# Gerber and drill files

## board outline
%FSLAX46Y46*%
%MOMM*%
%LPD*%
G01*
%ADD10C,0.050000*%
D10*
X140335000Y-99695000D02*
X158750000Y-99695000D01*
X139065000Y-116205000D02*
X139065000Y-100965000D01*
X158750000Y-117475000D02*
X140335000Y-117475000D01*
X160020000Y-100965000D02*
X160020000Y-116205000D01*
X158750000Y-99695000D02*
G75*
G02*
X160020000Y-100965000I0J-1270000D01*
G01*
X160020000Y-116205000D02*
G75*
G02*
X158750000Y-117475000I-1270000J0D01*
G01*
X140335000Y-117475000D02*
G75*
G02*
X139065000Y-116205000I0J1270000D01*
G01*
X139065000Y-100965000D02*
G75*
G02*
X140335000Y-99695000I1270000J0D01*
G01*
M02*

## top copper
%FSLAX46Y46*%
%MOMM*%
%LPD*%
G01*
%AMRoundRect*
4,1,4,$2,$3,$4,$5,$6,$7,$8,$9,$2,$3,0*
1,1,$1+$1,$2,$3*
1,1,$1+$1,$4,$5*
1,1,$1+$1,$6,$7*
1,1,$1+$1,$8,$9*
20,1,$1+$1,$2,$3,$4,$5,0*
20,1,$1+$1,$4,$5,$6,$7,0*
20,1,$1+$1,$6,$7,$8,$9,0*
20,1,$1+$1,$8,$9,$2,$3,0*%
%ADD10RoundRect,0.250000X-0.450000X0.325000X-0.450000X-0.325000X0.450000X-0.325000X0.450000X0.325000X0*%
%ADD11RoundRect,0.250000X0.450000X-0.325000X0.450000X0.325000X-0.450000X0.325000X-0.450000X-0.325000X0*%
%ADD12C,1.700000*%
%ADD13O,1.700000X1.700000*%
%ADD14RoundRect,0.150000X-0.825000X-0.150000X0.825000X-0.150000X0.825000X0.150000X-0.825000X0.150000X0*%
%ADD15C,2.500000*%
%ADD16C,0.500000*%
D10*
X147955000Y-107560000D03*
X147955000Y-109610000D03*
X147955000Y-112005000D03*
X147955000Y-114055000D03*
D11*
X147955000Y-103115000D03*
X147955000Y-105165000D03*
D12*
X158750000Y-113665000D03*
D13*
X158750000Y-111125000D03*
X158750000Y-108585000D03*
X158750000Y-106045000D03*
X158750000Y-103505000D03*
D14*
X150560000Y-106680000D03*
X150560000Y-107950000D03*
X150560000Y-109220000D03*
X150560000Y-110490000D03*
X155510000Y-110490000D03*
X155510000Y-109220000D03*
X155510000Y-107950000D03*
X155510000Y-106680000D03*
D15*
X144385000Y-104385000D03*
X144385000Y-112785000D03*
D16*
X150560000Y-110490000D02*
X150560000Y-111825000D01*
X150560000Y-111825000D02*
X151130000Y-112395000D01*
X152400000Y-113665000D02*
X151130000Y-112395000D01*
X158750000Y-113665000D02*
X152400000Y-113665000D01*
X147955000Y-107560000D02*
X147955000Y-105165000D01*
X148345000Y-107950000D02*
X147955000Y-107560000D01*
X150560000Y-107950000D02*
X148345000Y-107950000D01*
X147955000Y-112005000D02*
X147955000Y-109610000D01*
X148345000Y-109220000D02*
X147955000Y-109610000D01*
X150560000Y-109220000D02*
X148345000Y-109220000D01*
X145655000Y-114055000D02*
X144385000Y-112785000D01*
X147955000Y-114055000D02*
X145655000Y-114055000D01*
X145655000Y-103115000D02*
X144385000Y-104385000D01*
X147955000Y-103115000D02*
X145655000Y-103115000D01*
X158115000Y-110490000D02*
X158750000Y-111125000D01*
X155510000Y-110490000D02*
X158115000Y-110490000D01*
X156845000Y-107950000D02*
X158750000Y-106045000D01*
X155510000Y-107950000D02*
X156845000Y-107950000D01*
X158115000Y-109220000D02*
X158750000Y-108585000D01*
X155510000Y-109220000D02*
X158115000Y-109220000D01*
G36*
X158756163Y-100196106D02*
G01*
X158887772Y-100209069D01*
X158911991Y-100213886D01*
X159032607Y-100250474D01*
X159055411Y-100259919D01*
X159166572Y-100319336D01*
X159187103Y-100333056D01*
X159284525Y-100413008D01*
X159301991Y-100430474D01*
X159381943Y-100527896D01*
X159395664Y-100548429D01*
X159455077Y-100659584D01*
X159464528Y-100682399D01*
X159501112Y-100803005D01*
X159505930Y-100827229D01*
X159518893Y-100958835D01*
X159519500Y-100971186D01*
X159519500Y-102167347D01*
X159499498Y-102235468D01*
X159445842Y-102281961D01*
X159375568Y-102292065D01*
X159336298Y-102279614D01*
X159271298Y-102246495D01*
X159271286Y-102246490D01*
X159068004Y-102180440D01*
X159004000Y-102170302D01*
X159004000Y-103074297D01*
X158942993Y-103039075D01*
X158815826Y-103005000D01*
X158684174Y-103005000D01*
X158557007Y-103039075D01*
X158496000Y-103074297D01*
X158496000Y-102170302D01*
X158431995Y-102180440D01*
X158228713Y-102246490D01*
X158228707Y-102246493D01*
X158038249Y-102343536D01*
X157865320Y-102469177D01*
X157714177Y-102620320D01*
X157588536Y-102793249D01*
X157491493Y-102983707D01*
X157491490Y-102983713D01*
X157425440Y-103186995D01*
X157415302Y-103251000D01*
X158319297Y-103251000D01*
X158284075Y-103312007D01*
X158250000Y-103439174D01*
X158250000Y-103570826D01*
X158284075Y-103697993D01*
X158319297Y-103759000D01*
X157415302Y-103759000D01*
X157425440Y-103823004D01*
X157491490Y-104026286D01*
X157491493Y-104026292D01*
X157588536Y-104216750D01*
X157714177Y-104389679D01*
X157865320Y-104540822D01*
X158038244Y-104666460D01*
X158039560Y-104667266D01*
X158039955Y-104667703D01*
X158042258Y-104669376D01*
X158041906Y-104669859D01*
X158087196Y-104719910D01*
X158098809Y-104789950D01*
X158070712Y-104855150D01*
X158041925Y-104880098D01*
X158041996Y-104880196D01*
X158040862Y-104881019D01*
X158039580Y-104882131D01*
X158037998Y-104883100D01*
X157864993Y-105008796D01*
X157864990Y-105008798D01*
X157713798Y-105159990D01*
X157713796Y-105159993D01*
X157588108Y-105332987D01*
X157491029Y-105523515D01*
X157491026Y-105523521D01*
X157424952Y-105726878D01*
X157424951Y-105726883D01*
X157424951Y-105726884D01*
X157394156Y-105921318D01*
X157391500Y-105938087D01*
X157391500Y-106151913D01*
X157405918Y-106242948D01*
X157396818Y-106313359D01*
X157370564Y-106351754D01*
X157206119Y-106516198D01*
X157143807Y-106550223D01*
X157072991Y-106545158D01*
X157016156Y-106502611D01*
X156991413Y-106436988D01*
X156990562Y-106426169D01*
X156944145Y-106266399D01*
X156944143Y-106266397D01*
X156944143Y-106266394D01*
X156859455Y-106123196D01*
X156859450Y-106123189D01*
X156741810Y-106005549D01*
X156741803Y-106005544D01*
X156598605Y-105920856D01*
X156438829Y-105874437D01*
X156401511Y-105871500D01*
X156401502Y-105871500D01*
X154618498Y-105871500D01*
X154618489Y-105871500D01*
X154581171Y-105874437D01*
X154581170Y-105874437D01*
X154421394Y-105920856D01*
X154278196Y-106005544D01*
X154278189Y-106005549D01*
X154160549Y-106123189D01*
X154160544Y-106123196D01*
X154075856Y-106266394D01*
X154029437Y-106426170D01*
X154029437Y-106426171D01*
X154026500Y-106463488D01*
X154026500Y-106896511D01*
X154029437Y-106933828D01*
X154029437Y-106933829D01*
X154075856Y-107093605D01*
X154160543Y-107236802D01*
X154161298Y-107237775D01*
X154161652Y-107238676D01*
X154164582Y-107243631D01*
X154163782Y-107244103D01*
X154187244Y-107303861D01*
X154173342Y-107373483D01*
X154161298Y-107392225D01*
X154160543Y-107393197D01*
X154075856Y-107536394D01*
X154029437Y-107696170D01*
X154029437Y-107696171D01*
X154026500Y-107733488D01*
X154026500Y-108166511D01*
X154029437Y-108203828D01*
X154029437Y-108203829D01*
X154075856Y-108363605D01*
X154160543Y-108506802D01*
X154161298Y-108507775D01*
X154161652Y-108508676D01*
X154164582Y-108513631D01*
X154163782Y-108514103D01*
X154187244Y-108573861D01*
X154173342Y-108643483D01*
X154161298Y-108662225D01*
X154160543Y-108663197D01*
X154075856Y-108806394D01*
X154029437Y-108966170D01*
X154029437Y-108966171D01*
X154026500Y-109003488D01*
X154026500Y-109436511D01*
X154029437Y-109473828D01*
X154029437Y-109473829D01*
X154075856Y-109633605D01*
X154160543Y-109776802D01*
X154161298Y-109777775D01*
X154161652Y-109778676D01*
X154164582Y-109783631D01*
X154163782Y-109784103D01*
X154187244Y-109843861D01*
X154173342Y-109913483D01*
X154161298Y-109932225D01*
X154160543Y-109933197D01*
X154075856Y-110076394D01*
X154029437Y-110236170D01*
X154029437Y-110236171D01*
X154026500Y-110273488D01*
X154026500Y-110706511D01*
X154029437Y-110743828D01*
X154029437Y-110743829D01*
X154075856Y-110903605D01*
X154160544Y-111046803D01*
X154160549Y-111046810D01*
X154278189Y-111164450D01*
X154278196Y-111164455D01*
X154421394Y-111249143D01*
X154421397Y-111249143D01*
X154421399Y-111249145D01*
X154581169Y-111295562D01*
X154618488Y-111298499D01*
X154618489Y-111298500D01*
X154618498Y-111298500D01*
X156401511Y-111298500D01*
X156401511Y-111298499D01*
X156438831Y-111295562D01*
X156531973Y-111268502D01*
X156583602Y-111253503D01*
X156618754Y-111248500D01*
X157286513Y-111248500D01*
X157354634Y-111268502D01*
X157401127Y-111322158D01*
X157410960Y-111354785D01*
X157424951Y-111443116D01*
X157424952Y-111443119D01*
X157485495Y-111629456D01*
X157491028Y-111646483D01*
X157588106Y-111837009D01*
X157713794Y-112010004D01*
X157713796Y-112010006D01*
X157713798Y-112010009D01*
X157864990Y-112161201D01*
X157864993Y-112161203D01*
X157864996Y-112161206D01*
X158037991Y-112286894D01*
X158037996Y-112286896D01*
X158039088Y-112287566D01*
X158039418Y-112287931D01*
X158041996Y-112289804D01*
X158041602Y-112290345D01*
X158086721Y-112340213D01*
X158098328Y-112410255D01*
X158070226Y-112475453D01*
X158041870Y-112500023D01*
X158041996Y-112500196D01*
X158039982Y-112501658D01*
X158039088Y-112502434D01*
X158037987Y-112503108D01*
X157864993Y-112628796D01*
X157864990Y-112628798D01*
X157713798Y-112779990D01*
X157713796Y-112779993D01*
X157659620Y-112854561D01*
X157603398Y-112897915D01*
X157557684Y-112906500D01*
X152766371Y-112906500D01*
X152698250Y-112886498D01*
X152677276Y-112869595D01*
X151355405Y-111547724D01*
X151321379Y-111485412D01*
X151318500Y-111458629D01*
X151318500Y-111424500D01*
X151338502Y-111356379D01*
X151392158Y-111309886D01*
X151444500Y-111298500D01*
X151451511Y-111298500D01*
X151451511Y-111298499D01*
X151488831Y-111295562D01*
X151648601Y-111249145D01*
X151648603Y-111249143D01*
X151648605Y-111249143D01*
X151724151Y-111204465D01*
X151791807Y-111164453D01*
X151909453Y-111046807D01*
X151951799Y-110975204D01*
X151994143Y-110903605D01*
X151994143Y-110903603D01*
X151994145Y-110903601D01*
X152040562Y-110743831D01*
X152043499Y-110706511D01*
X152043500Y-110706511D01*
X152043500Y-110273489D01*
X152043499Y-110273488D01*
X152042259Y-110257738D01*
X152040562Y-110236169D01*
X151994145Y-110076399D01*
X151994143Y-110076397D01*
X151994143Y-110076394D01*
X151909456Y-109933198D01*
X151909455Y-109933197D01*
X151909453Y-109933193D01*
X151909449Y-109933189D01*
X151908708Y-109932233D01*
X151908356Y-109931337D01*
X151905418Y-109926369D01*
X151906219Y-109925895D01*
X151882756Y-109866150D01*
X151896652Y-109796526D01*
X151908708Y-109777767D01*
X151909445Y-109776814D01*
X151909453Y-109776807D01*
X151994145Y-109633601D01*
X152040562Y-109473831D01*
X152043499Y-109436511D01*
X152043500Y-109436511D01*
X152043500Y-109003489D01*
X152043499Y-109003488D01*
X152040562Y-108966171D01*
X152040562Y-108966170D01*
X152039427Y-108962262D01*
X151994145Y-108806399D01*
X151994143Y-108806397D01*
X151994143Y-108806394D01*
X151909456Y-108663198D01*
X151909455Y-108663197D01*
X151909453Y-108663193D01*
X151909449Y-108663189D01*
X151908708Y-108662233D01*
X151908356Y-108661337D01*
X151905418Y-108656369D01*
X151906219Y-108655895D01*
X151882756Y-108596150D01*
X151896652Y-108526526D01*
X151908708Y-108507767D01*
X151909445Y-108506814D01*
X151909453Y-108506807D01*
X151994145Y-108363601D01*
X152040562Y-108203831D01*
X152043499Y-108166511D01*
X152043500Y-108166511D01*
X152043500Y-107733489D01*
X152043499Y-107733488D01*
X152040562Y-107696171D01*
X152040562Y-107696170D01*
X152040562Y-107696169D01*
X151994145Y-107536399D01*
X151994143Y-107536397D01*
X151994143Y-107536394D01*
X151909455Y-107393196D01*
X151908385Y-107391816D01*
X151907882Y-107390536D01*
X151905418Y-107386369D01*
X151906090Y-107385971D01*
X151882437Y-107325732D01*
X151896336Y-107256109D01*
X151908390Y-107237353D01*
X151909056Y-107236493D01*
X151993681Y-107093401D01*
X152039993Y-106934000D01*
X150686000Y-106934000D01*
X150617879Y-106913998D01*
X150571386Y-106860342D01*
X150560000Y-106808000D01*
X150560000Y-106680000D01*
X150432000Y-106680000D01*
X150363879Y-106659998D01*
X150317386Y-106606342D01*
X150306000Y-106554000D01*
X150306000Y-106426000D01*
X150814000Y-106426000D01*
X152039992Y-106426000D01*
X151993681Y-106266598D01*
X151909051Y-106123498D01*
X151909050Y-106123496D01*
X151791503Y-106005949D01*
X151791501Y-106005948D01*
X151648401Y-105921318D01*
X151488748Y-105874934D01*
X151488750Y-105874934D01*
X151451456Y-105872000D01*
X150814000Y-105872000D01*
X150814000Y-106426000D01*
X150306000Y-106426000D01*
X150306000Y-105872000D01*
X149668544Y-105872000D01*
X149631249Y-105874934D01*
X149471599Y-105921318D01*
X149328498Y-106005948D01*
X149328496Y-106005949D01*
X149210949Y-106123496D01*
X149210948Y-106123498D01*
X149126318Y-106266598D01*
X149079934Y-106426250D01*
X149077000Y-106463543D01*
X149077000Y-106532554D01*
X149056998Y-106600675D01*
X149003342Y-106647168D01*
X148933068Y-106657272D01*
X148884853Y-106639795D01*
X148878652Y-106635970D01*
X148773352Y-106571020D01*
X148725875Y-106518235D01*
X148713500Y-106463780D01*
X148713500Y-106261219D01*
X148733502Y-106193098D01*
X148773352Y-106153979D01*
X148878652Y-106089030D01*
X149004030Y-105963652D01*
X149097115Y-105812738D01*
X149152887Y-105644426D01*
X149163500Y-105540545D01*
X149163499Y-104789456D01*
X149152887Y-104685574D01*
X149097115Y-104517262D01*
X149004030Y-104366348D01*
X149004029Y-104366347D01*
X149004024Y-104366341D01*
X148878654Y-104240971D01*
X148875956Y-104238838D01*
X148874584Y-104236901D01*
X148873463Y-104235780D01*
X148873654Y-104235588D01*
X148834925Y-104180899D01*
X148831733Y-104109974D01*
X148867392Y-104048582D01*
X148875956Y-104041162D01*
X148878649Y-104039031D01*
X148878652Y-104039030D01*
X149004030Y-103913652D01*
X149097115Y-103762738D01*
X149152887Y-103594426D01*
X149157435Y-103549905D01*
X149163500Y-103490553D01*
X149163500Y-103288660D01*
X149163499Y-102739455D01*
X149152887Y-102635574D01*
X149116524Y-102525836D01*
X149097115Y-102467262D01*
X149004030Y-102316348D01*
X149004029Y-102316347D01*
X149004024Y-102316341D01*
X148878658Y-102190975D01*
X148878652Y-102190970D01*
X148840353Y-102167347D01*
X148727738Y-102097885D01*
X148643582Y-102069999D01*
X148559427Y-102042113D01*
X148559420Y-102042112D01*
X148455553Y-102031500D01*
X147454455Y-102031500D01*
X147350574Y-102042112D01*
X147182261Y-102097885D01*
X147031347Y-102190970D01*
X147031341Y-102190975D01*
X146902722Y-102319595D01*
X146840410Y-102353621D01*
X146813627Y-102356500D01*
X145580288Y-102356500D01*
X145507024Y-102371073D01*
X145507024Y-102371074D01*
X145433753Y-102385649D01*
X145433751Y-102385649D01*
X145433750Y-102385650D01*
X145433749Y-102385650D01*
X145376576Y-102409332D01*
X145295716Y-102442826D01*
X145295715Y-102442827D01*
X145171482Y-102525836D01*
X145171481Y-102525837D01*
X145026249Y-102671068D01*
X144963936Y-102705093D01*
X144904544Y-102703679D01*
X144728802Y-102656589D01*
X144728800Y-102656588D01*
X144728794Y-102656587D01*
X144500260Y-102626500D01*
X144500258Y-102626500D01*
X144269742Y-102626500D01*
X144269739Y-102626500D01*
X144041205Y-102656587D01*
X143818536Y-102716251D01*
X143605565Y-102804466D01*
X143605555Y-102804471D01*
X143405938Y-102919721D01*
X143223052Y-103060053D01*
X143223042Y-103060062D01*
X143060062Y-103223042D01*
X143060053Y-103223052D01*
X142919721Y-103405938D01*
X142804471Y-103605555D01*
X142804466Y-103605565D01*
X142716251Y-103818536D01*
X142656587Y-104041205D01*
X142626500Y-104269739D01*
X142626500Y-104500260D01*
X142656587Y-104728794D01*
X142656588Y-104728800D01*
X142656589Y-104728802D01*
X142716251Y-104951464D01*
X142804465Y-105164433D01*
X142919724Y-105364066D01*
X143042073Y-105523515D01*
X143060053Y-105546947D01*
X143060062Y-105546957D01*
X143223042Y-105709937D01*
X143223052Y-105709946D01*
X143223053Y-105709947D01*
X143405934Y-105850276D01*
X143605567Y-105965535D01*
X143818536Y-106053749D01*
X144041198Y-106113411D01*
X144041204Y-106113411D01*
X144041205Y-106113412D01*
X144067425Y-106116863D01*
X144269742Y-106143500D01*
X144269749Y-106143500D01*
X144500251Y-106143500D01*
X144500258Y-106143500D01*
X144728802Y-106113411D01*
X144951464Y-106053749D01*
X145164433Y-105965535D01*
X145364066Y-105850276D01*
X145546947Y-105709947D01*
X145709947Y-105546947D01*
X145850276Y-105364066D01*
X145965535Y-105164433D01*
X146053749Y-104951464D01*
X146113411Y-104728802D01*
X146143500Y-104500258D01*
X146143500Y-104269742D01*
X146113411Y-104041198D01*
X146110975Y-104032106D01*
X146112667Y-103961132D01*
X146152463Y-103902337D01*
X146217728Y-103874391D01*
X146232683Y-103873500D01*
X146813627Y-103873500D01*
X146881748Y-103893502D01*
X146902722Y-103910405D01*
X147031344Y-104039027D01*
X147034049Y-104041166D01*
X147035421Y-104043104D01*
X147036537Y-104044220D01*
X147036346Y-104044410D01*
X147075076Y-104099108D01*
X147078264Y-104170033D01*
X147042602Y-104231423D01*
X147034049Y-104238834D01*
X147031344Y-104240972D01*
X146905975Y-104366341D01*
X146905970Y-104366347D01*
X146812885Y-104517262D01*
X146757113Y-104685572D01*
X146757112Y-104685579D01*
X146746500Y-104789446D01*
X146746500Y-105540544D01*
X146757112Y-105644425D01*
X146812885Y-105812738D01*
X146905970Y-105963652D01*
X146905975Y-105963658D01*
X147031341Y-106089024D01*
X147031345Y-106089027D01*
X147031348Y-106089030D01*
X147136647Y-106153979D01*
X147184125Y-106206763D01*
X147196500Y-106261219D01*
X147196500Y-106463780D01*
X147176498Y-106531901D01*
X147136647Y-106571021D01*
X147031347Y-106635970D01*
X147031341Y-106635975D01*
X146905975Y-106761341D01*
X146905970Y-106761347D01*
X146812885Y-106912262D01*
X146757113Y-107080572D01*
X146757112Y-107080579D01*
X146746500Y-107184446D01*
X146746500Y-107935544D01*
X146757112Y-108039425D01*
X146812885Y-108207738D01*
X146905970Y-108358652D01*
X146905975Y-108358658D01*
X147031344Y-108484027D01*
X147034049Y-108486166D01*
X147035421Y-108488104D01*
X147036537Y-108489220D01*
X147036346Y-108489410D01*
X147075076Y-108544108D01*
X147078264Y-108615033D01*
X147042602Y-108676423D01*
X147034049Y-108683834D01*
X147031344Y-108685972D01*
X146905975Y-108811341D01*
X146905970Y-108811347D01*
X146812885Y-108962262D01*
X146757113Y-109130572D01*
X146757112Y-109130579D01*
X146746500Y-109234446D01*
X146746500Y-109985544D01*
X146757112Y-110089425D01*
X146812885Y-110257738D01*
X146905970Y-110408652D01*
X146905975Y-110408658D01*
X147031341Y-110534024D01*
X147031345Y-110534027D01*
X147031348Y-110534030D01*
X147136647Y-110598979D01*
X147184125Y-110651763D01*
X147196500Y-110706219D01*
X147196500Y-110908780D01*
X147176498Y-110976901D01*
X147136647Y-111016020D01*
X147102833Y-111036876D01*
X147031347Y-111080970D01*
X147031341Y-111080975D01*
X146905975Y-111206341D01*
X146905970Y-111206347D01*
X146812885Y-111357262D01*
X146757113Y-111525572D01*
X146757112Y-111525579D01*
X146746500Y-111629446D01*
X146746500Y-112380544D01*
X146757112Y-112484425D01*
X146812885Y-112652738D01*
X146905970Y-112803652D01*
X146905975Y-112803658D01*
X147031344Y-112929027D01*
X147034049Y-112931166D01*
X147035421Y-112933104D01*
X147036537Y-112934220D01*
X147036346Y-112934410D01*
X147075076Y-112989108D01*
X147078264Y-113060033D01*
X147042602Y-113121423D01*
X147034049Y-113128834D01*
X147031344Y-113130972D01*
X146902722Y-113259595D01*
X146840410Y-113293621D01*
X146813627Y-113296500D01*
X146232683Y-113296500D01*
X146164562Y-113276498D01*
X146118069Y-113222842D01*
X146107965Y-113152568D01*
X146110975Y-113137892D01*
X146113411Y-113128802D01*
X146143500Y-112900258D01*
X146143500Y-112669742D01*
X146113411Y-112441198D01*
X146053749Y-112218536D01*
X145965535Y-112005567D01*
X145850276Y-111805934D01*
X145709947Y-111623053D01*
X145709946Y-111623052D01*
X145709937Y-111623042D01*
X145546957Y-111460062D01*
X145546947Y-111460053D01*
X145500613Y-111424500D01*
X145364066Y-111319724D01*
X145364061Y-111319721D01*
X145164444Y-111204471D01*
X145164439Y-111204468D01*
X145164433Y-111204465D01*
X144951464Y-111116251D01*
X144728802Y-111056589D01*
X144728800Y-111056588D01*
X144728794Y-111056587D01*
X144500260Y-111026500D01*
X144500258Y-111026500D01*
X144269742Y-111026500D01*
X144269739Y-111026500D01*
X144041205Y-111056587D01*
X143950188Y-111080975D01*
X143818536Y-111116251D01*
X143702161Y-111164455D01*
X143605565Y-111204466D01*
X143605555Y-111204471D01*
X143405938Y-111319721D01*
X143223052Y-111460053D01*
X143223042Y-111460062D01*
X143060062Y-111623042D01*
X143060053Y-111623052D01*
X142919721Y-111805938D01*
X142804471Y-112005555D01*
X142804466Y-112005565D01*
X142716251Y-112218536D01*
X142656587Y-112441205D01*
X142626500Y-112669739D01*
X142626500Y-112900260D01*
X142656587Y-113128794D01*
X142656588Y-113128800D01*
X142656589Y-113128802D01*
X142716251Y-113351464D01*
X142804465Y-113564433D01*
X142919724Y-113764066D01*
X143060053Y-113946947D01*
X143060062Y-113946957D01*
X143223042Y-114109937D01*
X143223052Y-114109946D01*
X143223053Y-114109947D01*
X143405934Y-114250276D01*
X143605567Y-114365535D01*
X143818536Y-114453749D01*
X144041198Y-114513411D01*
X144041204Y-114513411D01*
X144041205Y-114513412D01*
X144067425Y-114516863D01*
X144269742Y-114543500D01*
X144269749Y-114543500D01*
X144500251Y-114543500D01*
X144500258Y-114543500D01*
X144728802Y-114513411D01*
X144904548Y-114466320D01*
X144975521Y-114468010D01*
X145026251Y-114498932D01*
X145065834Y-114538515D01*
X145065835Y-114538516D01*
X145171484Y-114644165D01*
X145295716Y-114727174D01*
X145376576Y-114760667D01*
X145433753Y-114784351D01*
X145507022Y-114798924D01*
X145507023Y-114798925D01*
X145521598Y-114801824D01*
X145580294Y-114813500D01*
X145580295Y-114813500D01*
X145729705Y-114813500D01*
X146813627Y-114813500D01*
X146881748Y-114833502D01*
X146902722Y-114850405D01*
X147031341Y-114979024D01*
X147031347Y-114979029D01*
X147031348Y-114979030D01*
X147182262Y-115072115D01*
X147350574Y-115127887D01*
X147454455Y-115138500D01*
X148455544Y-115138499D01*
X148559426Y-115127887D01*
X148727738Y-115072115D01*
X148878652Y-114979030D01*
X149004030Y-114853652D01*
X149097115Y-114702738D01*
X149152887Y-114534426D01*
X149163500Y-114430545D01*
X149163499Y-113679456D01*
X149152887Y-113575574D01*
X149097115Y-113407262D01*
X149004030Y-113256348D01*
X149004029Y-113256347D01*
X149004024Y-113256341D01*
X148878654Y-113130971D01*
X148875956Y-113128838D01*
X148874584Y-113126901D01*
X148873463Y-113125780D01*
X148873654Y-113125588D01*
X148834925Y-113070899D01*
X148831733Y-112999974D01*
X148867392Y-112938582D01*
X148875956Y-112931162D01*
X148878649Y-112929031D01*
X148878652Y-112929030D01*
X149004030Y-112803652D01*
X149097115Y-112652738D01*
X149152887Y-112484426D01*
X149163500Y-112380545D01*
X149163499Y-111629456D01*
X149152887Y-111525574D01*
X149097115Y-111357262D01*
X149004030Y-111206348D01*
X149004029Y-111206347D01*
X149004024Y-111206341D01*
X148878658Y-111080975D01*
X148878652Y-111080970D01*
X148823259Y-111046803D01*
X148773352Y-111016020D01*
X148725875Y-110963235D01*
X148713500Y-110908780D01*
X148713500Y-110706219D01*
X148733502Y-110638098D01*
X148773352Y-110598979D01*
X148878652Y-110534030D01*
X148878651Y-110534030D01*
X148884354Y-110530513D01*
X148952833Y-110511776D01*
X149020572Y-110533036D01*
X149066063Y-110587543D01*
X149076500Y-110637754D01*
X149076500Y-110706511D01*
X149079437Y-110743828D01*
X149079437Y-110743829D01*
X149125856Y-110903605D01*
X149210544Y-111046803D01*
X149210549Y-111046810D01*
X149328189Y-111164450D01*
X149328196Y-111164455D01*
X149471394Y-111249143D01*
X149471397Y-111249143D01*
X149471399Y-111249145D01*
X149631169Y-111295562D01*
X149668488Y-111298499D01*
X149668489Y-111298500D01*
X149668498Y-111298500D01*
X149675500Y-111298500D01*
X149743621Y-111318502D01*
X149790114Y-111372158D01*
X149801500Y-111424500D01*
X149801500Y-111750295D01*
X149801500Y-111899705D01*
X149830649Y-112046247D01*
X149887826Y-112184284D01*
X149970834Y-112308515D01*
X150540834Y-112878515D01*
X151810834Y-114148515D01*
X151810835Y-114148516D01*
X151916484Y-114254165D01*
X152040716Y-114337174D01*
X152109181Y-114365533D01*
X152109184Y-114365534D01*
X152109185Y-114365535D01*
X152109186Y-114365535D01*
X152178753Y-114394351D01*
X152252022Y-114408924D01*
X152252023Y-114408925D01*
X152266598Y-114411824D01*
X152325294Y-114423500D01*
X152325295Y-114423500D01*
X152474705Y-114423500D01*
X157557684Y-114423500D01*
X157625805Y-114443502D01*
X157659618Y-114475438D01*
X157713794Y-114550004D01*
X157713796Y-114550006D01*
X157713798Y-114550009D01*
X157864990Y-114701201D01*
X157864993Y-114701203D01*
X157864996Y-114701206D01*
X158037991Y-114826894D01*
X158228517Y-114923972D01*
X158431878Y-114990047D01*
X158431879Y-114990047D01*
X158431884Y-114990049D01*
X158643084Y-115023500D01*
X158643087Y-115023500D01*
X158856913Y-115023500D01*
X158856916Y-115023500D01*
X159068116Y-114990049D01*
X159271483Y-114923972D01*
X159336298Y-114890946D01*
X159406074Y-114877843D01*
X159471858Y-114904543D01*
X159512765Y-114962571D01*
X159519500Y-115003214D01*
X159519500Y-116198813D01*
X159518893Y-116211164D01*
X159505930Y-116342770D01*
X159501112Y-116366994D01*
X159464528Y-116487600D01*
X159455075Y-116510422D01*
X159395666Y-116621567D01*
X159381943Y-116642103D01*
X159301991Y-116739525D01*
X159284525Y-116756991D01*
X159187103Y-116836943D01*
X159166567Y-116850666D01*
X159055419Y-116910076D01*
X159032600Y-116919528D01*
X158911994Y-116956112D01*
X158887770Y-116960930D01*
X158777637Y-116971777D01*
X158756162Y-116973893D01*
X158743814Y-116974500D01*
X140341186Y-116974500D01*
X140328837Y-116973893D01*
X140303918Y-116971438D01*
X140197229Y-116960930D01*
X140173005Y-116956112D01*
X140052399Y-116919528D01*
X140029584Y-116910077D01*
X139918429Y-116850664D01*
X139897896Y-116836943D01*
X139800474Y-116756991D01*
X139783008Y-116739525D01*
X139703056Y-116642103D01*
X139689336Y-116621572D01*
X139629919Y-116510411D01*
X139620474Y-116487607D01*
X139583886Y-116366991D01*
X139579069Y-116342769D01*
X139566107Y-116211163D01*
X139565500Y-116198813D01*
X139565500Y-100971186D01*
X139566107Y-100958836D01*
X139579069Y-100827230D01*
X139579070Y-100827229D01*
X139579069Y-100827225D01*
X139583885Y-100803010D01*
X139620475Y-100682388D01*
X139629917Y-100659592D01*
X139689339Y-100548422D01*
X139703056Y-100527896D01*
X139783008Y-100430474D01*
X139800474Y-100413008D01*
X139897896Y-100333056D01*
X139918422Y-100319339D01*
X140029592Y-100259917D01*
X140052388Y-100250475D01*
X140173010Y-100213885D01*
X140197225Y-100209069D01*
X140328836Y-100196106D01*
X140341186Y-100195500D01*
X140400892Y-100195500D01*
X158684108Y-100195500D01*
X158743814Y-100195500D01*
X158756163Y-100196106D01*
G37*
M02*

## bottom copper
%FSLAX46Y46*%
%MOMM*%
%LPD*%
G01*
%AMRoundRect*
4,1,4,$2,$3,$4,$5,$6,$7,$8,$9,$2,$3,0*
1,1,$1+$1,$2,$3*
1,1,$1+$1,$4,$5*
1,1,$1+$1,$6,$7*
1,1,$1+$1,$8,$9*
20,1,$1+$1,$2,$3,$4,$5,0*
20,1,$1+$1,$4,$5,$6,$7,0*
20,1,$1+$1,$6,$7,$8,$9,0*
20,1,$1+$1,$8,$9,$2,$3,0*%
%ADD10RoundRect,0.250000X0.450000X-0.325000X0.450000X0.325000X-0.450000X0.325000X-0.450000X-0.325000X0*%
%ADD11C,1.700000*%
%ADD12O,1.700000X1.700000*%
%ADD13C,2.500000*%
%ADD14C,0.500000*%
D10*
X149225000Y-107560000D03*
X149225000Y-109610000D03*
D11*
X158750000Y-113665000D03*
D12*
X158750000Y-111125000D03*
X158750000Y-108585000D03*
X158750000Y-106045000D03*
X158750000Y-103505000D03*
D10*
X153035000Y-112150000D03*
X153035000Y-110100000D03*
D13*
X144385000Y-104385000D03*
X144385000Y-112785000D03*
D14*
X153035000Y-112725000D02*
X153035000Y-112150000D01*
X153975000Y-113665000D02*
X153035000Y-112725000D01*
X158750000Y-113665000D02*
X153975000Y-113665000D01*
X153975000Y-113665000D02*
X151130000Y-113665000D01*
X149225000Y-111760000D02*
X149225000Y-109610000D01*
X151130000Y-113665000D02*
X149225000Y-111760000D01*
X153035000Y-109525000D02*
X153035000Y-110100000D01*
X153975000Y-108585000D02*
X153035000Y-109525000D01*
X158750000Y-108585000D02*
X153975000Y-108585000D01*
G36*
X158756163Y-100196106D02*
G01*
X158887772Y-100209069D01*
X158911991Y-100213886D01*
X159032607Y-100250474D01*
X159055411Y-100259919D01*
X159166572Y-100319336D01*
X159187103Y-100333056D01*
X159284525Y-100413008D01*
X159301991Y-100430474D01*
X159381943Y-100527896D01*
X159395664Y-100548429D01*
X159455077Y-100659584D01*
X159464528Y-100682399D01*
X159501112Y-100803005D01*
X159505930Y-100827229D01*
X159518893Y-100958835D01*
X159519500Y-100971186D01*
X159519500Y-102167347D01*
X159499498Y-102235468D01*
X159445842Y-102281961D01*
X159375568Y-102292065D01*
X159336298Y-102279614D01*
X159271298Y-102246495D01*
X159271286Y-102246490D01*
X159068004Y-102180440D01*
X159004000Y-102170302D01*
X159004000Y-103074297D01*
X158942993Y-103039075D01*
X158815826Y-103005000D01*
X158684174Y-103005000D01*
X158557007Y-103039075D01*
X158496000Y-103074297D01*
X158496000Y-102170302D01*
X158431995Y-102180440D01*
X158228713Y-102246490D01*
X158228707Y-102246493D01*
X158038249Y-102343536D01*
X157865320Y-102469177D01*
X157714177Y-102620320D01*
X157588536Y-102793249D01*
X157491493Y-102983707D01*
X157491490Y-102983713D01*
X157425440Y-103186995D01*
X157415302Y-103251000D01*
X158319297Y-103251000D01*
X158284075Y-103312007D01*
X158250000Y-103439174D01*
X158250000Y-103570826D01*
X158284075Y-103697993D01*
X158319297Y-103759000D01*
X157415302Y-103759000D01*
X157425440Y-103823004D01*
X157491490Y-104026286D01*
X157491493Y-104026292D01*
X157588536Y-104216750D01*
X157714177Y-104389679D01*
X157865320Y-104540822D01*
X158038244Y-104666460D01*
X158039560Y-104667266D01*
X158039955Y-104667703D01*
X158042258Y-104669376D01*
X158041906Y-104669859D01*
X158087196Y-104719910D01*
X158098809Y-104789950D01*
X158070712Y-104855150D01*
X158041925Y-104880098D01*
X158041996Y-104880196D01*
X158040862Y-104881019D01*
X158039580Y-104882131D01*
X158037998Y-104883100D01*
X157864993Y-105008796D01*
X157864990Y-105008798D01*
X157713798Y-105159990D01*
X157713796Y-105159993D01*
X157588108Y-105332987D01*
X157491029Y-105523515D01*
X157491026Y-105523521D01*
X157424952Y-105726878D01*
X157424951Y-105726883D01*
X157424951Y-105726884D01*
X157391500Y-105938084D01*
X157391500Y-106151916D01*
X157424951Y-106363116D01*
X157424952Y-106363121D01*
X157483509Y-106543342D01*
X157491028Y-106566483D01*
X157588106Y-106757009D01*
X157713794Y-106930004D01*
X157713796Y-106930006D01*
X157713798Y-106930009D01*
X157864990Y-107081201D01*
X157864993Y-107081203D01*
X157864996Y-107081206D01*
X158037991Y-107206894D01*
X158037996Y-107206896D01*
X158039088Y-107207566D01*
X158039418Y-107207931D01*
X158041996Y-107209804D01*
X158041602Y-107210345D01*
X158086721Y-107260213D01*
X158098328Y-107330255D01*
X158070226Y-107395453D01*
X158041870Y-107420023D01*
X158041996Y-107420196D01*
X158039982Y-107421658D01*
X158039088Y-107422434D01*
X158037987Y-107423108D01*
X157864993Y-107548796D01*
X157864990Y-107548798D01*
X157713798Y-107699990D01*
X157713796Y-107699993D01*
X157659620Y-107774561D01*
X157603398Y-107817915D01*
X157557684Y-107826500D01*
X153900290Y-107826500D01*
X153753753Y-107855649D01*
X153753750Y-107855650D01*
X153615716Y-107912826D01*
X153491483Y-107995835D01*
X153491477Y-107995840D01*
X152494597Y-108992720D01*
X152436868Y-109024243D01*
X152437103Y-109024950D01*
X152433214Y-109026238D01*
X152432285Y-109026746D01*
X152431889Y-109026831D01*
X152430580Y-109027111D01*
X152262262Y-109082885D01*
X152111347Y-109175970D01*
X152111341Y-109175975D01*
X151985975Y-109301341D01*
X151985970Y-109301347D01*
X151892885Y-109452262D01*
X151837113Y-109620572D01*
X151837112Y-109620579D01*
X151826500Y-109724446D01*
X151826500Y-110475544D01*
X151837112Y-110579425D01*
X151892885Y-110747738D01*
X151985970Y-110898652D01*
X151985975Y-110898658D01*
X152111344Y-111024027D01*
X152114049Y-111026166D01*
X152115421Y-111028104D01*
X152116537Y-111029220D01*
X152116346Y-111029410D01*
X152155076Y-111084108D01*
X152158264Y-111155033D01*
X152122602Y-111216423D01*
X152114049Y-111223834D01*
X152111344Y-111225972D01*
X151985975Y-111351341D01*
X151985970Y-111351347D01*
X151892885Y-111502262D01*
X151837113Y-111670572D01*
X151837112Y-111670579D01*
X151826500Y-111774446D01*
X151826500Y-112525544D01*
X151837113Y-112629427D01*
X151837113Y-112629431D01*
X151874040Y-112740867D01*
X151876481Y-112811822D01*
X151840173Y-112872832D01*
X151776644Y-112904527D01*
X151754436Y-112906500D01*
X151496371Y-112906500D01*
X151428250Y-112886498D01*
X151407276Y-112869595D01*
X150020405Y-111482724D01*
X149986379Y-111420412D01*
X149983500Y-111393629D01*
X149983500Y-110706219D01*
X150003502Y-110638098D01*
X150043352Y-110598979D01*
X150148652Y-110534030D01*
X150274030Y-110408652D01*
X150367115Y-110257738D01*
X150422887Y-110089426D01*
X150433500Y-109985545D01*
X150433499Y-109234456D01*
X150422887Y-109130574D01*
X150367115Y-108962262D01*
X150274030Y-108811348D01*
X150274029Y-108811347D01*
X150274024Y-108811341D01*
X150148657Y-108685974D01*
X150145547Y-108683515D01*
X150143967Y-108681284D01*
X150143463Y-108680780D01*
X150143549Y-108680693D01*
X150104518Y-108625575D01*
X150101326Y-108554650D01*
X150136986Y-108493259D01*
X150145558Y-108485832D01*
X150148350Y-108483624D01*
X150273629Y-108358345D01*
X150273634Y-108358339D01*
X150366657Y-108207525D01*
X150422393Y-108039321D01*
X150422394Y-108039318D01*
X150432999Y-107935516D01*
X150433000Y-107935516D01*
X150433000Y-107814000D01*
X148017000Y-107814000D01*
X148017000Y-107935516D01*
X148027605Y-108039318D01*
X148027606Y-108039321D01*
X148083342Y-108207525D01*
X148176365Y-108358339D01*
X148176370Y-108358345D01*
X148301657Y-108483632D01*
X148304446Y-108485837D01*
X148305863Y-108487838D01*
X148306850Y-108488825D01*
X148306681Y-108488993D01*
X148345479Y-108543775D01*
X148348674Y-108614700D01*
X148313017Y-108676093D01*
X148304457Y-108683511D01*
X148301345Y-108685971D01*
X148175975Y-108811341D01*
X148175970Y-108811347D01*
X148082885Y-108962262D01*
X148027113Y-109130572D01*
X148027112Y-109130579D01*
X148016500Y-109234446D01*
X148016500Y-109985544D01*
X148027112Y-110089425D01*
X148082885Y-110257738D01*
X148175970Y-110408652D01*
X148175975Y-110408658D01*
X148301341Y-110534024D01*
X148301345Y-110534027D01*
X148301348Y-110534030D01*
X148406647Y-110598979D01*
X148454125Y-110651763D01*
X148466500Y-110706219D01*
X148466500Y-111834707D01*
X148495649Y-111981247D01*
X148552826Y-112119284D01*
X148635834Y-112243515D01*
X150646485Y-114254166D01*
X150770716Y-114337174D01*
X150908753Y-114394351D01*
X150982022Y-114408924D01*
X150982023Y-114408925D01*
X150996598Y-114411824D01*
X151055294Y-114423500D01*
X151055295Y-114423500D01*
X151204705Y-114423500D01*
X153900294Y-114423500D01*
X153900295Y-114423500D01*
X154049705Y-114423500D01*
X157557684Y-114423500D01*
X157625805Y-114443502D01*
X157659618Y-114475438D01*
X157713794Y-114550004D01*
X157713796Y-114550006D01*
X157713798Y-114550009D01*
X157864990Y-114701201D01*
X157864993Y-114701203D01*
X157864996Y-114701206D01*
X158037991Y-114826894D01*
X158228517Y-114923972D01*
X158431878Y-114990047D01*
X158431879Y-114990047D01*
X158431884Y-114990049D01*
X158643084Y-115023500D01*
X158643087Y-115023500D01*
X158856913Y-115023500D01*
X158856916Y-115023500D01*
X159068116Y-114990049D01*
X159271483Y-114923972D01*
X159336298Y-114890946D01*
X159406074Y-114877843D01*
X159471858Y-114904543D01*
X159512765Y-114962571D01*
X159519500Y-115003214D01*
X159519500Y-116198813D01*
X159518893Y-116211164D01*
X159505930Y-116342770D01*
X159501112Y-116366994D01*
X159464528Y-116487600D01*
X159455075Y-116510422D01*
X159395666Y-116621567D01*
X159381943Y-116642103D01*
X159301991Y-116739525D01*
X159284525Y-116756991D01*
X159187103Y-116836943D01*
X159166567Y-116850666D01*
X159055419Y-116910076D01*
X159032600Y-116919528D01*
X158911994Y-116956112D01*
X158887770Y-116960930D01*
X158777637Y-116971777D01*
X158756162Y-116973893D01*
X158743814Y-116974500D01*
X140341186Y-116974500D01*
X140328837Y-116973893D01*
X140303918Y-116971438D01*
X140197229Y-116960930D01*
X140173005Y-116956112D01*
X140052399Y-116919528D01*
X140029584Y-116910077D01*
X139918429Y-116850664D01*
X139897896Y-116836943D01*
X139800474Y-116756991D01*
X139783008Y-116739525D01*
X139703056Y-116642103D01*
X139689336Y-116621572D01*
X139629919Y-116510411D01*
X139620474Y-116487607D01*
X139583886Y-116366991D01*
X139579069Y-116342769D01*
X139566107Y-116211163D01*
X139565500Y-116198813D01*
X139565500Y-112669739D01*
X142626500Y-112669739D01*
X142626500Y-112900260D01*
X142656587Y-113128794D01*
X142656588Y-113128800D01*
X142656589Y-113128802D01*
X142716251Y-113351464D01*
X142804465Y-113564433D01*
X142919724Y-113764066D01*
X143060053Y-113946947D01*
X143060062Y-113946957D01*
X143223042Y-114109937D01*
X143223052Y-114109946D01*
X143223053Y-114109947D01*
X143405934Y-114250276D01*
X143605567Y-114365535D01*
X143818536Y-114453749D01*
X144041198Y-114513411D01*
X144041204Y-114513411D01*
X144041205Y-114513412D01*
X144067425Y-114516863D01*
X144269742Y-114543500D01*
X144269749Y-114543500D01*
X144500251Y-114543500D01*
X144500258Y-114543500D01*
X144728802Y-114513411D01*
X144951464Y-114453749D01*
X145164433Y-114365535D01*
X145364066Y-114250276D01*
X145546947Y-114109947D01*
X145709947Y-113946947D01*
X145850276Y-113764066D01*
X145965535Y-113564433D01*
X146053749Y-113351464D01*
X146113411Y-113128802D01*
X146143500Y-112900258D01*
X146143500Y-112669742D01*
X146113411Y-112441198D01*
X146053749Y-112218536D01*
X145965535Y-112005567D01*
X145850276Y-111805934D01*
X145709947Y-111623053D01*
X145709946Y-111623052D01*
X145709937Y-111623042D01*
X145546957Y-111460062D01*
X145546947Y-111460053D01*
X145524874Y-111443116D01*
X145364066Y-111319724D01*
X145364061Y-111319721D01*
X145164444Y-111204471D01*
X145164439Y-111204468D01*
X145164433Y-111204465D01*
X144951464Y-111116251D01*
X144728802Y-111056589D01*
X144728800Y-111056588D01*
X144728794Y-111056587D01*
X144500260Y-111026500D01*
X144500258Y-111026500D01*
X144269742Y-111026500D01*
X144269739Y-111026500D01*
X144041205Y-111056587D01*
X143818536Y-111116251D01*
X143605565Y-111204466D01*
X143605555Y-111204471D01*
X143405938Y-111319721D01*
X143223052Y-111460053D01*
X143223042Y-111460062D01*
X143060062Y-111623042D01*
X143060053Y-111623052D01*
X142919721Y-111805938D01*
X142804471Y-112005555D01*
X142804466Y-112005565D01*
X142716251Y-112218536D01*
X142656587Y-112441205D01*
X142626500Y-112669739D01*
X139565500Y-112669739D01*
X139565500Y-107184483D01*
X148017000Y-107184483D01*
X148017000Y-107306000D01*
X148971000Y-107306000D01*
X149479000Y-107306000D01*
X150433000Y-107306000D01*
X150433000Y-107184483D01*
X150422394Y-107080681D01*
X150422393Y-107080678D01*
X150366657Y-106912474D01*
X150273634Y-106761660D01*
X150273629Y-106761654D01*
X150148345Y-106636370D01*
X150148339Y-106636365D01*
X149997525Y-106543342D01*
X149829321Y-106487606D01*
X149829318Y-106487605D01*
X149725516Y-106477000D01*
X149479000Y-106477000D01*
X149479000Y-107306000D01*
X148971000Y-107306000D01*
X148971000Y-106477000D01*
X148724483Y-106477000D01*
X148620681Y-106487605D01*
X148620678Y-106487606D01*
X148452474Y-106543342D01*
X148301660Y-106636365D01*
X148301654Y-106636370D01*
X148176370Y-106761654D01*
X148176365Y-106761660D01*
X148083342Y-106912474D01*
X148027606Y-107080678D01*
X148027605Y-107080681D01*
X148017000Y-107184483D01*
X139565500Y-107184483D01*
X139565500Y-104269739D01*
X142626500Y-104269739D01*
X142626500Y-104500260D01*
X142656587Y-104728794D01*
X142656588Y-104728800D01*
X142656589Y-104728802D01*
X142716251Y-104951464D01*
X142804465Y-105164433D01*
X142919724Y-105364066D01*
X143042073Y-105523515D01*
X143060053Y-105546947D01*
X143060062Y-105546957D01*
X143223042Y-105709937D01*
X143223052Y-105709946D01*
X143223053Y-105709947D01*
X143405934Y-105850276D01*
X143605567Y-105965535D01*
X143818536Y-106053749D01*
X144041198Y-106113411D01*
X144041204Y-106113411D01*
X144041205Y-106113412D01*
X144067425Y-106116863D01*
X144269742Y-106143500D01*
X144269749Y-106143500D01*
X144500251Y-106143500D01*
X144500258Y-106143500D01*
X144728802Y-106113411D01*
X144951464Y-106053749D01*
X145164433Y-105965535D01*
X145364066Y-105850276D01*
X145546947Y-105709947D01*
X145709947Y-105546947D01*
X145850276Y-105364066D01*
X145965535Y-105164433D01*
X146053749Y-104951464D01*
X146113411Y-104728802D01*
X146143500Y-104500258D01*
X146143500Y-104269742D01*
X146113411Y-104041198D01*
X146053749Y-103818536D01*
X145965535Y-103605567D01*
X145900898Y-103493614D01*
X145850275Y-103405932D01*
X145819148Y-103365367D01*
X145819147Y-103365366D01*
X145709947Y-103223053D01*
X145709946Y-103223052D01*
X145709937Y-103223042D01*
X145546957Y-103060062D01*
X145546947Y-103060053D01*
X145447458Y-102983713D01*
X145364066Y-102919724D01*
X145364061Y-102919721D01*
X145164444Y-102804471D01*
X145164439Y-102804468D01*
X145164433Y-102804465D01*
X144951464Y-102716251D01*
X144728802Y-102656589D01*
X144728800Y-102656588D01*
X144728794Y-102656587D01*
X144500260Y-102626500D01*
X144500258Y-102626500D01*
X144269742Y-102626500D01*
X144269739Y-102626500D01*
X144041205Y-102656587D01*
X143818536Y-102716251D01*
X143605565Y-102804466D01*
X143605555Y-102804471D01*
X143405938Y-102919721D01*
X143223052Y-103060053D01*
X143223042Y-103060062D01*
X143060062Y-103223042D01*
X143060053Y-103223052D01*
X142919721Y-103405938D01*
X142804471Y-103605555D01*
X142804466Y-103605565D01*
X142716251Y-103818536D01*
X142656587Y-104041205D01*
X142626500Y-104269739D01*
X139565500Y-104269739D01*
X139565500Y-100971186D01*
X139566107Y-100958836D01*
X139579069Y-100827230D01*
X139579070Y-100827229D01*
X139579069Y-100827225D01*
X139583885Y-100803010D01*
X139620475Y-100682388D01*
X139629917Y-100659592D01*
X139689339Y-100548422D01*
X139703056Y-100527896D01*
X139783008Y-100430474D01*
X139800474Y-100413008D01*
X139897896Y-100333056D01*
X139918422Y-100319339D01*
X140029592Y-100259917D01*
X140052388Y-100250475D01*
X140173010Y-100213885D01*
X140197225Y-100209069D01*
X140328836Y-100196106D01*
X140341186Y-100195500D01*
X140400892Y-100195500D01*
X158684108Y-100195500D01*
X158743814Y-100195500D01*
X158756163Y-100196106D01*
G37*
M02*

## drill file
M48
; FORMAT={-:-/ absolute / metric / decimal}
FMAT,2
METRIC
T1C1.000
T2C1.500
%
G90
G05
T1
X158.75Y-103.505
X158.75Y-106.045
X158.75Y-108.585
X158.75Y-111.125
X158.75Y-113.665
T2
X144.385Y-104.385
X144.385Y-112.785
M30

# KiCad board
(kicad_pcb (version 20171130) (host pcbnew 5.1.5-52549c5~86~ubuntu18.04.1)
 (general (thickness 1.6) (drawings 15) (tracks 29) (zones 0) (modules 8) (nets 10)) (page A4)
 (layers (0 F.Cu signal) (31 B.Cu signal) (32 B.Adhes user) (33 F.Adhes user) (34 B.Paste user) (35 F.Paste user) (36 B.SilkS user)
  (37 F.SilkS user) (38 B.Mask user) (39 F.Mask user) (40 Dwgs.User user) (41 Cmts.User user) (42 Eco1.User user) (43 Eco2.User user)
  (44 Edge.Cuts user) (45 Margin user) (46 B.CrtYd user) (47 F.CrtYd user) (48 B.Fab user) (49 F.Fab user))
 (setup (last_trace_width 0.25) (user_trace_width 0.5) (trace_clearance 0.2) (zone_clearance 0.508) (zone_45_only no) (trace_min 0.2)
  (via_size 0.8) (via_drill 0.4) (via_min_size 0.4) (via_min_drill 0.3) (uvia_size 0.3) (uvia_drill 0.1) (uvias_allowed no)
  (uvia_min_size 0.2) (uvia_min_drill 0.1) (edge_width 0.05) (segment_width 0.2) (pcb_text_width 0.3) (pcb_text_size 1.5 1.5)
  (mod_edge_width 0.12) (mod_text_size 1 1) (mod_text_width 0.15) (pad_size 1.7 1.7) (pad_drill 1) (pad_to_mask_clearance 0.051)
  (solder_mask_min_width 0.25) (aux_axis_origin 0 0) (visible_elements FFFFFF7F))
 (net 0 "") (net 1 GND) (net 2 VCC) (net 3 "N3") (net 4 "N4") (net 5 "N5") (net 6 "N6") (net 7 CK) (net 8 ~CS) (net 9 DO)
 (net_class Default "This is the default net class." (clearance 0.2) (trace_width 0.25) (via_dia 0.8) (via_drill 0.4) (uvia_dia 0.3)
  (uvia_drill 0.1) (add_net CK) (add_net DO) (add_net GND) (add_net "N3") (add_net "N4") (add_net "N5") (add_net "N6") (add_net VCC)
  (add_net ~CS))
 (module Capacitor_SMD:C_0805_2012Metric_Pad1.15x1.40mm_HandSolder (layer B.Cu) (at 149.225 108.585 90)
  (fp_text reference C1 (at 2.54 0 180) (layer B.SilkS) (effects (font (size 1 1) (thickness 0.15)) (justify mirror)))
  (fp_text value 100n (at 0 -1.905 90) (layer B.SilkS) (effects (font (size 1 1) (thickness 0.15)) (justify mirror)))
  (pad 2 smd roundrect (at 1.025 0 90) (size 1.15 1.4) (layers B.Cu B.Paste B.Mask) (roundrect_rratio 0.217391) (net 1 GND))
  (pad 1 smd roundrect (at -1.025 0 90) (size 1.15 1.4) (layers B.Cu B.Paste B.Mask) (roundrect_rratio 0.217391) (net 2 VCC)))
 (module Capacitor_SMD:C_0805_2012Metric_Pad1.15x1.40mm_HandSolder (layer F.Cu) (at 147.955 108.585 270)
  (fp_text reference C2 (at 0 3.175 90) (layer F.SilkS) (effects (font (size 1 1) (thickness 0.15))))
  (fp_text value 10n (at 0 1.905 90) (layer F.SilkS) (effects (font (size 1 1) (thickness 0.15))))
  (pad 1 smd roundrect (at -1.025 0 270) (size 1.15 1.4) (layers F.Cu F.Paste F.Mask) (roundrect_rratio 0.217391) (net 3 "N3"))
  (pad 2 smd roundrect (at 1.025 0 270) (size 1.15 1.4) (layers F.Cu F.Paste F.Mask) (roundrect_rratio 0.217391) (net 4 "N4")))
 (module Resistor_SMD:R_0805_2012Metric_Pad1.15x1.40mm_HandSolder (layer F.Cu) (at 147.955 113.03 270)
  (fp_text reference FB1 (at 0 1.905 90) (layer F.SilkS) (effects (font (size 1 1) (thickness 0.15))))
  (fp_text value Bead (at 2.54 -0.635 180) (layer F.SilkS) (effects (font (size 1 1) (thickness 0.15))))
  (pad 1 smd roundrect (at -1.025 0 270) (size 1.15 1.4) (layers F.Cu F.Paste F.Mask) (roundrect_rratio 0.217391) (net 4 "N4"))
  (pad 2 smd roundrect (at 1.025 0 270) (size 1.15 1.4) (layers F.Cu F.Paste F.Mask) (roundrect_rratio 0.217391) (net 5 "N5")))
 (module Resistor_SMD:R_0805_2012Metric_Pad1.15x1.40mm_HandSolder (layer F.Cu) (at 147.955 104.14 90)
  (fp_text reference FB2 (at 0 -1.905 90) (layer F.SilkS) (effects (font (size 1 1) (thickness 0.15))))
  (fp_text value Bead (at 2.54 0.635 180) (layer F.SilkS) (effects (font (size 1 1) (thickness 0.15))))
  (pad 2 smd roundrect (at 1.025 0 90) (size 1.15 1.4) (layers F.Cu F.Paste F.Mask) (roundrect_rratio 0.217391) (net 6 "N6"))
  (pad 1 smd roundrect (at -1.025 0 90) (size 1.15 1.4) (layers F.Cu F.Paste F.Mask) (roundrect_rratio 0.217391) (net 3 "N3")))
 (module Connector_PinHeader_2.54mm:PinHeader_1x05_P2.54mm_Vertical (layer F.Cu) (at 158.75 113.665 180)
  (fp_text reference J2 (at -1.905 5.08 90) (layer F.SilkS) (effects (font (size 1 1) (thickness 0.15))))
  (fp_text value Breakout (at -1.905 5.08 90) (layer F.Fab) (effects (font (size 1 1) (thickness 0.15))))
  (pad 1 thru_hole circle (at 0 0 180) (size 1.7 1.7) (drill 1) (layers *.Cu *.Mask) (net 2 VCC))
  (pad 2 thru_hole oval (at 0 2.54 180) (size 1.7 1.7) (drill 1) (layers *.Cu *.Mask) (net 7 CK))
  (pad 3 thru_hole oval (at 0 5.08 180) (size 1.7 1.7) (drill 1) (layers *.Cu *.Mask) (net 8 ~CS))
  (pad 4 thru_hole oval (at 0 7.62 180) (size 1.7 1.7) (drill 1) (layers *.Cu *.Mask) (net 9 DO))
  (pad 5 thru_hole oval (at 0 10.16 180) (size 1.7 1.7) (drill 1) (layers *.Cu *.Mask) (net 1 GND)))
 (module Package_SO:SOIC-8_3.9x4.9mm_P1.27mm (layer F.Cu) (at 153.035 108.585)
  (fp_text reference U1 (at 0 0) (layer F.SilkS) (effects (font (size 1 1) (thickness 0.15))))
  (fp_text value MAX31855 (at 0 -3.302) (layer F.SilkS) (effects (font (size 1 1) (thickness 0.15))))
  (pad 1 smd roundrect (at -2.475 -1.905) (size 1.95 0.6) (layers F.Cu F.Paste F.Mask) (roundrect_rratio 0.25) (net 1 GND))
  (pad 2 smd roundrect (at -2.475 -0.635) (size 1.95 0.6) (layers F.Cu F.Paste F.Mask) (roundrect_rratio 0.25) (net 3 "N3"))
  (pad 3 smd roundrect (at -2.475 0.635) (size 1.95 0.6) (layers F.Cu F.Paste F.Mask) (roundrect_rratio 0.25) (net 4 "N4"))
  (pad 4 smd roundrect (at -2.475 1.905) (size 1.95 0.6) (layers F.Cu F.Paste F.Mask) (roundrect_rratio 0.25) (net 2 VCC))
  (pad 5 smd roundrect (at 2.475 1.905) (size 1.95 0.6) (layers F.Cu F.Paste F.Mask) (roundrect_rratio 0.25) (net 7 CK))
  (pad 6 smd roundrect (at 2.475 0.635) (size 1.95 0.6) (layers F.Cu F.Paste F.Mask) (roundrect_rratio 0.25) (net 8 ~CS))
  (pad 7 smd roundrect (at 2.475 -0.635) (size 1.95 0.6) (layers F.Cu F.Paste F.Mask) (roundrect_rratio 0.25) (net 9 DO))
  (pad 8 smd roundrect (at 2.475 -1.905) (size 1.95 0.6) (layers F.Cu F.Paste F.Mask) (roundrect_rratio 0.25)))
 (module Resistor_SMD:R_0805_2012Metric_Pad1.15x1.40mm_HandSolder (layer B.Cu) (at 153.035 111.125 90)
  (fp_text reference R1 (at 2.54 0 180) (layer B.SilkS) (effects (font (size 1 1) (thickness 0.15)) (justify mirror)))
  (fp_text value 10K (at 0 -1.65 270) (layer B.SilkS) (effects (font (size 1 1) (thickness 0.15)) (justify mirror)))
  (pad 1 smd roundrect (at -1.025 0 90) (size 1.15 1.4) (layers B.Cu B.Paste B.Mask) (roundrect_rratio 0.217391) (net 2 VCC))
  (pad 2 smd roundrect (at 1.025 0 90) (size 1.15 1.4) (layers B.Cu B.Paste B.Mask) (roundrect_rratio 0.217391) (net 8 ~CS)))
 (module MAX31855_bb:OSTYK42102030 (layer F.Cu) (at 140.335 108.585 270)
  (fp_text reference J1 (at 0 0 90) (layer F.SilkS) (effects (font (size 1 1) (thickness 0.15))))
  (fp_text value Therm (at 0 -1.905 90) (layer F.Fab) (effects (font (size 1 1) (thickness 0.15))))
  (pad 1 thru_hole circle (at -4.2 -4.05 270) (size 2.5 2.5) (drill 1.5) (layers *.Cu *.Mask) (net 6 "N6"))
  (pad 2 thru_hole circle (at 4.2 -4.05 270) (size 2.5 2.5) (drill 1.5) (layers *.Cu *.Mask) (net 5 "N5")))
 (gr_line (start 140.335 99.695) (end 158.75 99.695) (layer Edge.Cuts) (width 0.05))
 (gr_line (start 139.065 116.205) (end 139.065 100.965) (layer Edge.Cuts) (width 0.05))
 (gr_line (start 158.75 117.475) (end 140.335 117.475) (layer Edge.Cuts) (width 0.05))
 (gr_line (start 160.02 100.965) (end 160.02 116.205) (layer Edge.Cuts) (width 0.05))
 (gr_arc (start 158.75 100.965) (end 160.02 100.965) (angle -90) (layer Edge.Cuts) (width 0.05))
 (gr_arc (start 158.75 116.205) (end 158.75 117.475) (angle -90) (layer Edge.Cuts) (width 0.05))
 (gr_arc (start 140.335 116.205) (end 139.065 116.205) (angle -90) (layer Edge.Cuts) (width 0.05))
 (gr_arc (start 140.335 100.965) (end 140.335 99.695) (angle -90) (layer Edge.Cuts) (width 0.05))
 (segment (start 150.56 110.49) (end 150.56 111.825) (width 0.5) (layer F.Cu) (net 2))
 (segment (start 150.56 111.825) (end 151.13 112.395) (width 0.5) (layer F.Cu) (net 2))
 (segment (start 152.4 113.665) (end 151.13 112.395) (width 0.5) (layer F.Cu) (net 2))
 (segment (start 158.75 113.665) (end 152.4 113.665) (width 0.5) (layer F.Cu) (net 2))
 (segment (start 153.035 112.725) (end 153.035 112.15) (width 0.5) (layer B.Cu) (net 2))
 (segment (start 153.975 113.665) (end 153.035 112.725) (width 0.5) (layer B.Cu) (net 2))
 (segment (start 158.75 113.665) (end 153.975 113.665) (width 0.5) (layer B.Cu) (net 2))
 (segment (start 153.975 113.665) (end 151.13 113.665) (width 0.5) (layer B.Cu) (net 2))
 (segment (start 149.225 111.76) (end 149.225 109.61) (width 0.5) (layer B.Cu) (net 2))
 (segment (start 151.13 113.665) (end 149.225 111.76) (width 0.5) (layer B.Cu) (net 2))
 (segment (start 147.955 107.56) (end 147.955 105.165) (width 0.5) (layer F.Cu) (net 3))
 (segment (start 148.345 107.95) (end 147.955 107.56) (width 0.5) (layer F.Cu) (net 3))
 (segment (start 150.56 107.95) (end 148.345 107.95) (width 0.5) (layer F.Cu) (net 3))
 (segment (start 147.955 112.005) (end 147.955 109.61) (width 0.5) (layer F.Cu) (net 4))
 (segment (start 148.345 109.22) (end 147.955 109.61) (width 0.5) (layer F.Cu) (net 4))
 (segment (start 150.56 109.22) (end 148.345 109.22) (width 0.5) (layer F.Cu) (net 4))
 (segment (start 145.655 114.055) (end 144.385 112.785) (width 0.5) (layer F.Cu) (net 5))
 (segment (start 147.955 114.055) (end 145.655 114.055) (width 0.5) (layer F.Cu) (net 5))
 (segment (start 145.655 103.115) (end 144.385 104.385) (width 0.5) (layer F.Cu) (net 6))
 (segment (start 147.955 103.115) (end 145.655 103.115) (width 0.5) (layer F.Cu) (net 6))
 (segment (start 158.115 110.49) (end 158.75 111.125) (width 0.5) (layer F.Cu) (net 7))
 (segment (start 155.51 110.49) (end 158.115 110.49) (width 0.5) (layer F.Cu) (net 7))
 (segment (start 156.845 107.95) (end 158.75 106.045) (width 0.5) (layer F.Cu) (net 9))
 (segment (start 155.51 107.95) (end 156.845 107.95) (width 0.5) (layer F.Cu) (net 9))
 (segment (start 158.115 109.22) (end 158.75 108.585) (width 0.5) (layer F.Cu) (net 8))
 (segment (start 155.51 109.22) (end 158.115 109.22) (width 0.5) (layer F.Cu) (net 8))
 (segment (start 153.035 109.525) (end 153.035 110.1) (width 0.5) (layer B.Cu) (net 8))
 (segment (start 153.975 108.585) (end 153.035 109.525) (width 0.5) (layer B.Cu) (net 8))
 (segment (start 158.75 108.585) (end 153.975 108.585) (width 0.5) (layer B.Cu) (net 8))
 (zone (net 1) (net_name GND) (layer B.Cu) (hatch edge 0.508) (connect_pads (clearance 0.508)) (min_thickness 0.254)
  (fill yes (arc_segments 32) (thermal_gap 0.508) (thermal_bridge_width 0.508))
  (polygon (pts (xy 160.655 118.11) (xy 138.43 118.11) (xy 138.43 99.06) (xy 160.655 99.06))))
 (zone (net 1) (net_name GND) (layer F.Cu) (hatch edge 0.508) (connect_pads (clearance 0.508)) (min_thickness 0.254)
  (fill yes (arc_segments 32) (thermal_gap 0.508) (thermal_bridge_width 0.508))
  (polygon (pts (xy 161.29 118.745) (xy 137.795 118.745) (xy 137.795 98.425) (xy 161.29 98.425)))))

